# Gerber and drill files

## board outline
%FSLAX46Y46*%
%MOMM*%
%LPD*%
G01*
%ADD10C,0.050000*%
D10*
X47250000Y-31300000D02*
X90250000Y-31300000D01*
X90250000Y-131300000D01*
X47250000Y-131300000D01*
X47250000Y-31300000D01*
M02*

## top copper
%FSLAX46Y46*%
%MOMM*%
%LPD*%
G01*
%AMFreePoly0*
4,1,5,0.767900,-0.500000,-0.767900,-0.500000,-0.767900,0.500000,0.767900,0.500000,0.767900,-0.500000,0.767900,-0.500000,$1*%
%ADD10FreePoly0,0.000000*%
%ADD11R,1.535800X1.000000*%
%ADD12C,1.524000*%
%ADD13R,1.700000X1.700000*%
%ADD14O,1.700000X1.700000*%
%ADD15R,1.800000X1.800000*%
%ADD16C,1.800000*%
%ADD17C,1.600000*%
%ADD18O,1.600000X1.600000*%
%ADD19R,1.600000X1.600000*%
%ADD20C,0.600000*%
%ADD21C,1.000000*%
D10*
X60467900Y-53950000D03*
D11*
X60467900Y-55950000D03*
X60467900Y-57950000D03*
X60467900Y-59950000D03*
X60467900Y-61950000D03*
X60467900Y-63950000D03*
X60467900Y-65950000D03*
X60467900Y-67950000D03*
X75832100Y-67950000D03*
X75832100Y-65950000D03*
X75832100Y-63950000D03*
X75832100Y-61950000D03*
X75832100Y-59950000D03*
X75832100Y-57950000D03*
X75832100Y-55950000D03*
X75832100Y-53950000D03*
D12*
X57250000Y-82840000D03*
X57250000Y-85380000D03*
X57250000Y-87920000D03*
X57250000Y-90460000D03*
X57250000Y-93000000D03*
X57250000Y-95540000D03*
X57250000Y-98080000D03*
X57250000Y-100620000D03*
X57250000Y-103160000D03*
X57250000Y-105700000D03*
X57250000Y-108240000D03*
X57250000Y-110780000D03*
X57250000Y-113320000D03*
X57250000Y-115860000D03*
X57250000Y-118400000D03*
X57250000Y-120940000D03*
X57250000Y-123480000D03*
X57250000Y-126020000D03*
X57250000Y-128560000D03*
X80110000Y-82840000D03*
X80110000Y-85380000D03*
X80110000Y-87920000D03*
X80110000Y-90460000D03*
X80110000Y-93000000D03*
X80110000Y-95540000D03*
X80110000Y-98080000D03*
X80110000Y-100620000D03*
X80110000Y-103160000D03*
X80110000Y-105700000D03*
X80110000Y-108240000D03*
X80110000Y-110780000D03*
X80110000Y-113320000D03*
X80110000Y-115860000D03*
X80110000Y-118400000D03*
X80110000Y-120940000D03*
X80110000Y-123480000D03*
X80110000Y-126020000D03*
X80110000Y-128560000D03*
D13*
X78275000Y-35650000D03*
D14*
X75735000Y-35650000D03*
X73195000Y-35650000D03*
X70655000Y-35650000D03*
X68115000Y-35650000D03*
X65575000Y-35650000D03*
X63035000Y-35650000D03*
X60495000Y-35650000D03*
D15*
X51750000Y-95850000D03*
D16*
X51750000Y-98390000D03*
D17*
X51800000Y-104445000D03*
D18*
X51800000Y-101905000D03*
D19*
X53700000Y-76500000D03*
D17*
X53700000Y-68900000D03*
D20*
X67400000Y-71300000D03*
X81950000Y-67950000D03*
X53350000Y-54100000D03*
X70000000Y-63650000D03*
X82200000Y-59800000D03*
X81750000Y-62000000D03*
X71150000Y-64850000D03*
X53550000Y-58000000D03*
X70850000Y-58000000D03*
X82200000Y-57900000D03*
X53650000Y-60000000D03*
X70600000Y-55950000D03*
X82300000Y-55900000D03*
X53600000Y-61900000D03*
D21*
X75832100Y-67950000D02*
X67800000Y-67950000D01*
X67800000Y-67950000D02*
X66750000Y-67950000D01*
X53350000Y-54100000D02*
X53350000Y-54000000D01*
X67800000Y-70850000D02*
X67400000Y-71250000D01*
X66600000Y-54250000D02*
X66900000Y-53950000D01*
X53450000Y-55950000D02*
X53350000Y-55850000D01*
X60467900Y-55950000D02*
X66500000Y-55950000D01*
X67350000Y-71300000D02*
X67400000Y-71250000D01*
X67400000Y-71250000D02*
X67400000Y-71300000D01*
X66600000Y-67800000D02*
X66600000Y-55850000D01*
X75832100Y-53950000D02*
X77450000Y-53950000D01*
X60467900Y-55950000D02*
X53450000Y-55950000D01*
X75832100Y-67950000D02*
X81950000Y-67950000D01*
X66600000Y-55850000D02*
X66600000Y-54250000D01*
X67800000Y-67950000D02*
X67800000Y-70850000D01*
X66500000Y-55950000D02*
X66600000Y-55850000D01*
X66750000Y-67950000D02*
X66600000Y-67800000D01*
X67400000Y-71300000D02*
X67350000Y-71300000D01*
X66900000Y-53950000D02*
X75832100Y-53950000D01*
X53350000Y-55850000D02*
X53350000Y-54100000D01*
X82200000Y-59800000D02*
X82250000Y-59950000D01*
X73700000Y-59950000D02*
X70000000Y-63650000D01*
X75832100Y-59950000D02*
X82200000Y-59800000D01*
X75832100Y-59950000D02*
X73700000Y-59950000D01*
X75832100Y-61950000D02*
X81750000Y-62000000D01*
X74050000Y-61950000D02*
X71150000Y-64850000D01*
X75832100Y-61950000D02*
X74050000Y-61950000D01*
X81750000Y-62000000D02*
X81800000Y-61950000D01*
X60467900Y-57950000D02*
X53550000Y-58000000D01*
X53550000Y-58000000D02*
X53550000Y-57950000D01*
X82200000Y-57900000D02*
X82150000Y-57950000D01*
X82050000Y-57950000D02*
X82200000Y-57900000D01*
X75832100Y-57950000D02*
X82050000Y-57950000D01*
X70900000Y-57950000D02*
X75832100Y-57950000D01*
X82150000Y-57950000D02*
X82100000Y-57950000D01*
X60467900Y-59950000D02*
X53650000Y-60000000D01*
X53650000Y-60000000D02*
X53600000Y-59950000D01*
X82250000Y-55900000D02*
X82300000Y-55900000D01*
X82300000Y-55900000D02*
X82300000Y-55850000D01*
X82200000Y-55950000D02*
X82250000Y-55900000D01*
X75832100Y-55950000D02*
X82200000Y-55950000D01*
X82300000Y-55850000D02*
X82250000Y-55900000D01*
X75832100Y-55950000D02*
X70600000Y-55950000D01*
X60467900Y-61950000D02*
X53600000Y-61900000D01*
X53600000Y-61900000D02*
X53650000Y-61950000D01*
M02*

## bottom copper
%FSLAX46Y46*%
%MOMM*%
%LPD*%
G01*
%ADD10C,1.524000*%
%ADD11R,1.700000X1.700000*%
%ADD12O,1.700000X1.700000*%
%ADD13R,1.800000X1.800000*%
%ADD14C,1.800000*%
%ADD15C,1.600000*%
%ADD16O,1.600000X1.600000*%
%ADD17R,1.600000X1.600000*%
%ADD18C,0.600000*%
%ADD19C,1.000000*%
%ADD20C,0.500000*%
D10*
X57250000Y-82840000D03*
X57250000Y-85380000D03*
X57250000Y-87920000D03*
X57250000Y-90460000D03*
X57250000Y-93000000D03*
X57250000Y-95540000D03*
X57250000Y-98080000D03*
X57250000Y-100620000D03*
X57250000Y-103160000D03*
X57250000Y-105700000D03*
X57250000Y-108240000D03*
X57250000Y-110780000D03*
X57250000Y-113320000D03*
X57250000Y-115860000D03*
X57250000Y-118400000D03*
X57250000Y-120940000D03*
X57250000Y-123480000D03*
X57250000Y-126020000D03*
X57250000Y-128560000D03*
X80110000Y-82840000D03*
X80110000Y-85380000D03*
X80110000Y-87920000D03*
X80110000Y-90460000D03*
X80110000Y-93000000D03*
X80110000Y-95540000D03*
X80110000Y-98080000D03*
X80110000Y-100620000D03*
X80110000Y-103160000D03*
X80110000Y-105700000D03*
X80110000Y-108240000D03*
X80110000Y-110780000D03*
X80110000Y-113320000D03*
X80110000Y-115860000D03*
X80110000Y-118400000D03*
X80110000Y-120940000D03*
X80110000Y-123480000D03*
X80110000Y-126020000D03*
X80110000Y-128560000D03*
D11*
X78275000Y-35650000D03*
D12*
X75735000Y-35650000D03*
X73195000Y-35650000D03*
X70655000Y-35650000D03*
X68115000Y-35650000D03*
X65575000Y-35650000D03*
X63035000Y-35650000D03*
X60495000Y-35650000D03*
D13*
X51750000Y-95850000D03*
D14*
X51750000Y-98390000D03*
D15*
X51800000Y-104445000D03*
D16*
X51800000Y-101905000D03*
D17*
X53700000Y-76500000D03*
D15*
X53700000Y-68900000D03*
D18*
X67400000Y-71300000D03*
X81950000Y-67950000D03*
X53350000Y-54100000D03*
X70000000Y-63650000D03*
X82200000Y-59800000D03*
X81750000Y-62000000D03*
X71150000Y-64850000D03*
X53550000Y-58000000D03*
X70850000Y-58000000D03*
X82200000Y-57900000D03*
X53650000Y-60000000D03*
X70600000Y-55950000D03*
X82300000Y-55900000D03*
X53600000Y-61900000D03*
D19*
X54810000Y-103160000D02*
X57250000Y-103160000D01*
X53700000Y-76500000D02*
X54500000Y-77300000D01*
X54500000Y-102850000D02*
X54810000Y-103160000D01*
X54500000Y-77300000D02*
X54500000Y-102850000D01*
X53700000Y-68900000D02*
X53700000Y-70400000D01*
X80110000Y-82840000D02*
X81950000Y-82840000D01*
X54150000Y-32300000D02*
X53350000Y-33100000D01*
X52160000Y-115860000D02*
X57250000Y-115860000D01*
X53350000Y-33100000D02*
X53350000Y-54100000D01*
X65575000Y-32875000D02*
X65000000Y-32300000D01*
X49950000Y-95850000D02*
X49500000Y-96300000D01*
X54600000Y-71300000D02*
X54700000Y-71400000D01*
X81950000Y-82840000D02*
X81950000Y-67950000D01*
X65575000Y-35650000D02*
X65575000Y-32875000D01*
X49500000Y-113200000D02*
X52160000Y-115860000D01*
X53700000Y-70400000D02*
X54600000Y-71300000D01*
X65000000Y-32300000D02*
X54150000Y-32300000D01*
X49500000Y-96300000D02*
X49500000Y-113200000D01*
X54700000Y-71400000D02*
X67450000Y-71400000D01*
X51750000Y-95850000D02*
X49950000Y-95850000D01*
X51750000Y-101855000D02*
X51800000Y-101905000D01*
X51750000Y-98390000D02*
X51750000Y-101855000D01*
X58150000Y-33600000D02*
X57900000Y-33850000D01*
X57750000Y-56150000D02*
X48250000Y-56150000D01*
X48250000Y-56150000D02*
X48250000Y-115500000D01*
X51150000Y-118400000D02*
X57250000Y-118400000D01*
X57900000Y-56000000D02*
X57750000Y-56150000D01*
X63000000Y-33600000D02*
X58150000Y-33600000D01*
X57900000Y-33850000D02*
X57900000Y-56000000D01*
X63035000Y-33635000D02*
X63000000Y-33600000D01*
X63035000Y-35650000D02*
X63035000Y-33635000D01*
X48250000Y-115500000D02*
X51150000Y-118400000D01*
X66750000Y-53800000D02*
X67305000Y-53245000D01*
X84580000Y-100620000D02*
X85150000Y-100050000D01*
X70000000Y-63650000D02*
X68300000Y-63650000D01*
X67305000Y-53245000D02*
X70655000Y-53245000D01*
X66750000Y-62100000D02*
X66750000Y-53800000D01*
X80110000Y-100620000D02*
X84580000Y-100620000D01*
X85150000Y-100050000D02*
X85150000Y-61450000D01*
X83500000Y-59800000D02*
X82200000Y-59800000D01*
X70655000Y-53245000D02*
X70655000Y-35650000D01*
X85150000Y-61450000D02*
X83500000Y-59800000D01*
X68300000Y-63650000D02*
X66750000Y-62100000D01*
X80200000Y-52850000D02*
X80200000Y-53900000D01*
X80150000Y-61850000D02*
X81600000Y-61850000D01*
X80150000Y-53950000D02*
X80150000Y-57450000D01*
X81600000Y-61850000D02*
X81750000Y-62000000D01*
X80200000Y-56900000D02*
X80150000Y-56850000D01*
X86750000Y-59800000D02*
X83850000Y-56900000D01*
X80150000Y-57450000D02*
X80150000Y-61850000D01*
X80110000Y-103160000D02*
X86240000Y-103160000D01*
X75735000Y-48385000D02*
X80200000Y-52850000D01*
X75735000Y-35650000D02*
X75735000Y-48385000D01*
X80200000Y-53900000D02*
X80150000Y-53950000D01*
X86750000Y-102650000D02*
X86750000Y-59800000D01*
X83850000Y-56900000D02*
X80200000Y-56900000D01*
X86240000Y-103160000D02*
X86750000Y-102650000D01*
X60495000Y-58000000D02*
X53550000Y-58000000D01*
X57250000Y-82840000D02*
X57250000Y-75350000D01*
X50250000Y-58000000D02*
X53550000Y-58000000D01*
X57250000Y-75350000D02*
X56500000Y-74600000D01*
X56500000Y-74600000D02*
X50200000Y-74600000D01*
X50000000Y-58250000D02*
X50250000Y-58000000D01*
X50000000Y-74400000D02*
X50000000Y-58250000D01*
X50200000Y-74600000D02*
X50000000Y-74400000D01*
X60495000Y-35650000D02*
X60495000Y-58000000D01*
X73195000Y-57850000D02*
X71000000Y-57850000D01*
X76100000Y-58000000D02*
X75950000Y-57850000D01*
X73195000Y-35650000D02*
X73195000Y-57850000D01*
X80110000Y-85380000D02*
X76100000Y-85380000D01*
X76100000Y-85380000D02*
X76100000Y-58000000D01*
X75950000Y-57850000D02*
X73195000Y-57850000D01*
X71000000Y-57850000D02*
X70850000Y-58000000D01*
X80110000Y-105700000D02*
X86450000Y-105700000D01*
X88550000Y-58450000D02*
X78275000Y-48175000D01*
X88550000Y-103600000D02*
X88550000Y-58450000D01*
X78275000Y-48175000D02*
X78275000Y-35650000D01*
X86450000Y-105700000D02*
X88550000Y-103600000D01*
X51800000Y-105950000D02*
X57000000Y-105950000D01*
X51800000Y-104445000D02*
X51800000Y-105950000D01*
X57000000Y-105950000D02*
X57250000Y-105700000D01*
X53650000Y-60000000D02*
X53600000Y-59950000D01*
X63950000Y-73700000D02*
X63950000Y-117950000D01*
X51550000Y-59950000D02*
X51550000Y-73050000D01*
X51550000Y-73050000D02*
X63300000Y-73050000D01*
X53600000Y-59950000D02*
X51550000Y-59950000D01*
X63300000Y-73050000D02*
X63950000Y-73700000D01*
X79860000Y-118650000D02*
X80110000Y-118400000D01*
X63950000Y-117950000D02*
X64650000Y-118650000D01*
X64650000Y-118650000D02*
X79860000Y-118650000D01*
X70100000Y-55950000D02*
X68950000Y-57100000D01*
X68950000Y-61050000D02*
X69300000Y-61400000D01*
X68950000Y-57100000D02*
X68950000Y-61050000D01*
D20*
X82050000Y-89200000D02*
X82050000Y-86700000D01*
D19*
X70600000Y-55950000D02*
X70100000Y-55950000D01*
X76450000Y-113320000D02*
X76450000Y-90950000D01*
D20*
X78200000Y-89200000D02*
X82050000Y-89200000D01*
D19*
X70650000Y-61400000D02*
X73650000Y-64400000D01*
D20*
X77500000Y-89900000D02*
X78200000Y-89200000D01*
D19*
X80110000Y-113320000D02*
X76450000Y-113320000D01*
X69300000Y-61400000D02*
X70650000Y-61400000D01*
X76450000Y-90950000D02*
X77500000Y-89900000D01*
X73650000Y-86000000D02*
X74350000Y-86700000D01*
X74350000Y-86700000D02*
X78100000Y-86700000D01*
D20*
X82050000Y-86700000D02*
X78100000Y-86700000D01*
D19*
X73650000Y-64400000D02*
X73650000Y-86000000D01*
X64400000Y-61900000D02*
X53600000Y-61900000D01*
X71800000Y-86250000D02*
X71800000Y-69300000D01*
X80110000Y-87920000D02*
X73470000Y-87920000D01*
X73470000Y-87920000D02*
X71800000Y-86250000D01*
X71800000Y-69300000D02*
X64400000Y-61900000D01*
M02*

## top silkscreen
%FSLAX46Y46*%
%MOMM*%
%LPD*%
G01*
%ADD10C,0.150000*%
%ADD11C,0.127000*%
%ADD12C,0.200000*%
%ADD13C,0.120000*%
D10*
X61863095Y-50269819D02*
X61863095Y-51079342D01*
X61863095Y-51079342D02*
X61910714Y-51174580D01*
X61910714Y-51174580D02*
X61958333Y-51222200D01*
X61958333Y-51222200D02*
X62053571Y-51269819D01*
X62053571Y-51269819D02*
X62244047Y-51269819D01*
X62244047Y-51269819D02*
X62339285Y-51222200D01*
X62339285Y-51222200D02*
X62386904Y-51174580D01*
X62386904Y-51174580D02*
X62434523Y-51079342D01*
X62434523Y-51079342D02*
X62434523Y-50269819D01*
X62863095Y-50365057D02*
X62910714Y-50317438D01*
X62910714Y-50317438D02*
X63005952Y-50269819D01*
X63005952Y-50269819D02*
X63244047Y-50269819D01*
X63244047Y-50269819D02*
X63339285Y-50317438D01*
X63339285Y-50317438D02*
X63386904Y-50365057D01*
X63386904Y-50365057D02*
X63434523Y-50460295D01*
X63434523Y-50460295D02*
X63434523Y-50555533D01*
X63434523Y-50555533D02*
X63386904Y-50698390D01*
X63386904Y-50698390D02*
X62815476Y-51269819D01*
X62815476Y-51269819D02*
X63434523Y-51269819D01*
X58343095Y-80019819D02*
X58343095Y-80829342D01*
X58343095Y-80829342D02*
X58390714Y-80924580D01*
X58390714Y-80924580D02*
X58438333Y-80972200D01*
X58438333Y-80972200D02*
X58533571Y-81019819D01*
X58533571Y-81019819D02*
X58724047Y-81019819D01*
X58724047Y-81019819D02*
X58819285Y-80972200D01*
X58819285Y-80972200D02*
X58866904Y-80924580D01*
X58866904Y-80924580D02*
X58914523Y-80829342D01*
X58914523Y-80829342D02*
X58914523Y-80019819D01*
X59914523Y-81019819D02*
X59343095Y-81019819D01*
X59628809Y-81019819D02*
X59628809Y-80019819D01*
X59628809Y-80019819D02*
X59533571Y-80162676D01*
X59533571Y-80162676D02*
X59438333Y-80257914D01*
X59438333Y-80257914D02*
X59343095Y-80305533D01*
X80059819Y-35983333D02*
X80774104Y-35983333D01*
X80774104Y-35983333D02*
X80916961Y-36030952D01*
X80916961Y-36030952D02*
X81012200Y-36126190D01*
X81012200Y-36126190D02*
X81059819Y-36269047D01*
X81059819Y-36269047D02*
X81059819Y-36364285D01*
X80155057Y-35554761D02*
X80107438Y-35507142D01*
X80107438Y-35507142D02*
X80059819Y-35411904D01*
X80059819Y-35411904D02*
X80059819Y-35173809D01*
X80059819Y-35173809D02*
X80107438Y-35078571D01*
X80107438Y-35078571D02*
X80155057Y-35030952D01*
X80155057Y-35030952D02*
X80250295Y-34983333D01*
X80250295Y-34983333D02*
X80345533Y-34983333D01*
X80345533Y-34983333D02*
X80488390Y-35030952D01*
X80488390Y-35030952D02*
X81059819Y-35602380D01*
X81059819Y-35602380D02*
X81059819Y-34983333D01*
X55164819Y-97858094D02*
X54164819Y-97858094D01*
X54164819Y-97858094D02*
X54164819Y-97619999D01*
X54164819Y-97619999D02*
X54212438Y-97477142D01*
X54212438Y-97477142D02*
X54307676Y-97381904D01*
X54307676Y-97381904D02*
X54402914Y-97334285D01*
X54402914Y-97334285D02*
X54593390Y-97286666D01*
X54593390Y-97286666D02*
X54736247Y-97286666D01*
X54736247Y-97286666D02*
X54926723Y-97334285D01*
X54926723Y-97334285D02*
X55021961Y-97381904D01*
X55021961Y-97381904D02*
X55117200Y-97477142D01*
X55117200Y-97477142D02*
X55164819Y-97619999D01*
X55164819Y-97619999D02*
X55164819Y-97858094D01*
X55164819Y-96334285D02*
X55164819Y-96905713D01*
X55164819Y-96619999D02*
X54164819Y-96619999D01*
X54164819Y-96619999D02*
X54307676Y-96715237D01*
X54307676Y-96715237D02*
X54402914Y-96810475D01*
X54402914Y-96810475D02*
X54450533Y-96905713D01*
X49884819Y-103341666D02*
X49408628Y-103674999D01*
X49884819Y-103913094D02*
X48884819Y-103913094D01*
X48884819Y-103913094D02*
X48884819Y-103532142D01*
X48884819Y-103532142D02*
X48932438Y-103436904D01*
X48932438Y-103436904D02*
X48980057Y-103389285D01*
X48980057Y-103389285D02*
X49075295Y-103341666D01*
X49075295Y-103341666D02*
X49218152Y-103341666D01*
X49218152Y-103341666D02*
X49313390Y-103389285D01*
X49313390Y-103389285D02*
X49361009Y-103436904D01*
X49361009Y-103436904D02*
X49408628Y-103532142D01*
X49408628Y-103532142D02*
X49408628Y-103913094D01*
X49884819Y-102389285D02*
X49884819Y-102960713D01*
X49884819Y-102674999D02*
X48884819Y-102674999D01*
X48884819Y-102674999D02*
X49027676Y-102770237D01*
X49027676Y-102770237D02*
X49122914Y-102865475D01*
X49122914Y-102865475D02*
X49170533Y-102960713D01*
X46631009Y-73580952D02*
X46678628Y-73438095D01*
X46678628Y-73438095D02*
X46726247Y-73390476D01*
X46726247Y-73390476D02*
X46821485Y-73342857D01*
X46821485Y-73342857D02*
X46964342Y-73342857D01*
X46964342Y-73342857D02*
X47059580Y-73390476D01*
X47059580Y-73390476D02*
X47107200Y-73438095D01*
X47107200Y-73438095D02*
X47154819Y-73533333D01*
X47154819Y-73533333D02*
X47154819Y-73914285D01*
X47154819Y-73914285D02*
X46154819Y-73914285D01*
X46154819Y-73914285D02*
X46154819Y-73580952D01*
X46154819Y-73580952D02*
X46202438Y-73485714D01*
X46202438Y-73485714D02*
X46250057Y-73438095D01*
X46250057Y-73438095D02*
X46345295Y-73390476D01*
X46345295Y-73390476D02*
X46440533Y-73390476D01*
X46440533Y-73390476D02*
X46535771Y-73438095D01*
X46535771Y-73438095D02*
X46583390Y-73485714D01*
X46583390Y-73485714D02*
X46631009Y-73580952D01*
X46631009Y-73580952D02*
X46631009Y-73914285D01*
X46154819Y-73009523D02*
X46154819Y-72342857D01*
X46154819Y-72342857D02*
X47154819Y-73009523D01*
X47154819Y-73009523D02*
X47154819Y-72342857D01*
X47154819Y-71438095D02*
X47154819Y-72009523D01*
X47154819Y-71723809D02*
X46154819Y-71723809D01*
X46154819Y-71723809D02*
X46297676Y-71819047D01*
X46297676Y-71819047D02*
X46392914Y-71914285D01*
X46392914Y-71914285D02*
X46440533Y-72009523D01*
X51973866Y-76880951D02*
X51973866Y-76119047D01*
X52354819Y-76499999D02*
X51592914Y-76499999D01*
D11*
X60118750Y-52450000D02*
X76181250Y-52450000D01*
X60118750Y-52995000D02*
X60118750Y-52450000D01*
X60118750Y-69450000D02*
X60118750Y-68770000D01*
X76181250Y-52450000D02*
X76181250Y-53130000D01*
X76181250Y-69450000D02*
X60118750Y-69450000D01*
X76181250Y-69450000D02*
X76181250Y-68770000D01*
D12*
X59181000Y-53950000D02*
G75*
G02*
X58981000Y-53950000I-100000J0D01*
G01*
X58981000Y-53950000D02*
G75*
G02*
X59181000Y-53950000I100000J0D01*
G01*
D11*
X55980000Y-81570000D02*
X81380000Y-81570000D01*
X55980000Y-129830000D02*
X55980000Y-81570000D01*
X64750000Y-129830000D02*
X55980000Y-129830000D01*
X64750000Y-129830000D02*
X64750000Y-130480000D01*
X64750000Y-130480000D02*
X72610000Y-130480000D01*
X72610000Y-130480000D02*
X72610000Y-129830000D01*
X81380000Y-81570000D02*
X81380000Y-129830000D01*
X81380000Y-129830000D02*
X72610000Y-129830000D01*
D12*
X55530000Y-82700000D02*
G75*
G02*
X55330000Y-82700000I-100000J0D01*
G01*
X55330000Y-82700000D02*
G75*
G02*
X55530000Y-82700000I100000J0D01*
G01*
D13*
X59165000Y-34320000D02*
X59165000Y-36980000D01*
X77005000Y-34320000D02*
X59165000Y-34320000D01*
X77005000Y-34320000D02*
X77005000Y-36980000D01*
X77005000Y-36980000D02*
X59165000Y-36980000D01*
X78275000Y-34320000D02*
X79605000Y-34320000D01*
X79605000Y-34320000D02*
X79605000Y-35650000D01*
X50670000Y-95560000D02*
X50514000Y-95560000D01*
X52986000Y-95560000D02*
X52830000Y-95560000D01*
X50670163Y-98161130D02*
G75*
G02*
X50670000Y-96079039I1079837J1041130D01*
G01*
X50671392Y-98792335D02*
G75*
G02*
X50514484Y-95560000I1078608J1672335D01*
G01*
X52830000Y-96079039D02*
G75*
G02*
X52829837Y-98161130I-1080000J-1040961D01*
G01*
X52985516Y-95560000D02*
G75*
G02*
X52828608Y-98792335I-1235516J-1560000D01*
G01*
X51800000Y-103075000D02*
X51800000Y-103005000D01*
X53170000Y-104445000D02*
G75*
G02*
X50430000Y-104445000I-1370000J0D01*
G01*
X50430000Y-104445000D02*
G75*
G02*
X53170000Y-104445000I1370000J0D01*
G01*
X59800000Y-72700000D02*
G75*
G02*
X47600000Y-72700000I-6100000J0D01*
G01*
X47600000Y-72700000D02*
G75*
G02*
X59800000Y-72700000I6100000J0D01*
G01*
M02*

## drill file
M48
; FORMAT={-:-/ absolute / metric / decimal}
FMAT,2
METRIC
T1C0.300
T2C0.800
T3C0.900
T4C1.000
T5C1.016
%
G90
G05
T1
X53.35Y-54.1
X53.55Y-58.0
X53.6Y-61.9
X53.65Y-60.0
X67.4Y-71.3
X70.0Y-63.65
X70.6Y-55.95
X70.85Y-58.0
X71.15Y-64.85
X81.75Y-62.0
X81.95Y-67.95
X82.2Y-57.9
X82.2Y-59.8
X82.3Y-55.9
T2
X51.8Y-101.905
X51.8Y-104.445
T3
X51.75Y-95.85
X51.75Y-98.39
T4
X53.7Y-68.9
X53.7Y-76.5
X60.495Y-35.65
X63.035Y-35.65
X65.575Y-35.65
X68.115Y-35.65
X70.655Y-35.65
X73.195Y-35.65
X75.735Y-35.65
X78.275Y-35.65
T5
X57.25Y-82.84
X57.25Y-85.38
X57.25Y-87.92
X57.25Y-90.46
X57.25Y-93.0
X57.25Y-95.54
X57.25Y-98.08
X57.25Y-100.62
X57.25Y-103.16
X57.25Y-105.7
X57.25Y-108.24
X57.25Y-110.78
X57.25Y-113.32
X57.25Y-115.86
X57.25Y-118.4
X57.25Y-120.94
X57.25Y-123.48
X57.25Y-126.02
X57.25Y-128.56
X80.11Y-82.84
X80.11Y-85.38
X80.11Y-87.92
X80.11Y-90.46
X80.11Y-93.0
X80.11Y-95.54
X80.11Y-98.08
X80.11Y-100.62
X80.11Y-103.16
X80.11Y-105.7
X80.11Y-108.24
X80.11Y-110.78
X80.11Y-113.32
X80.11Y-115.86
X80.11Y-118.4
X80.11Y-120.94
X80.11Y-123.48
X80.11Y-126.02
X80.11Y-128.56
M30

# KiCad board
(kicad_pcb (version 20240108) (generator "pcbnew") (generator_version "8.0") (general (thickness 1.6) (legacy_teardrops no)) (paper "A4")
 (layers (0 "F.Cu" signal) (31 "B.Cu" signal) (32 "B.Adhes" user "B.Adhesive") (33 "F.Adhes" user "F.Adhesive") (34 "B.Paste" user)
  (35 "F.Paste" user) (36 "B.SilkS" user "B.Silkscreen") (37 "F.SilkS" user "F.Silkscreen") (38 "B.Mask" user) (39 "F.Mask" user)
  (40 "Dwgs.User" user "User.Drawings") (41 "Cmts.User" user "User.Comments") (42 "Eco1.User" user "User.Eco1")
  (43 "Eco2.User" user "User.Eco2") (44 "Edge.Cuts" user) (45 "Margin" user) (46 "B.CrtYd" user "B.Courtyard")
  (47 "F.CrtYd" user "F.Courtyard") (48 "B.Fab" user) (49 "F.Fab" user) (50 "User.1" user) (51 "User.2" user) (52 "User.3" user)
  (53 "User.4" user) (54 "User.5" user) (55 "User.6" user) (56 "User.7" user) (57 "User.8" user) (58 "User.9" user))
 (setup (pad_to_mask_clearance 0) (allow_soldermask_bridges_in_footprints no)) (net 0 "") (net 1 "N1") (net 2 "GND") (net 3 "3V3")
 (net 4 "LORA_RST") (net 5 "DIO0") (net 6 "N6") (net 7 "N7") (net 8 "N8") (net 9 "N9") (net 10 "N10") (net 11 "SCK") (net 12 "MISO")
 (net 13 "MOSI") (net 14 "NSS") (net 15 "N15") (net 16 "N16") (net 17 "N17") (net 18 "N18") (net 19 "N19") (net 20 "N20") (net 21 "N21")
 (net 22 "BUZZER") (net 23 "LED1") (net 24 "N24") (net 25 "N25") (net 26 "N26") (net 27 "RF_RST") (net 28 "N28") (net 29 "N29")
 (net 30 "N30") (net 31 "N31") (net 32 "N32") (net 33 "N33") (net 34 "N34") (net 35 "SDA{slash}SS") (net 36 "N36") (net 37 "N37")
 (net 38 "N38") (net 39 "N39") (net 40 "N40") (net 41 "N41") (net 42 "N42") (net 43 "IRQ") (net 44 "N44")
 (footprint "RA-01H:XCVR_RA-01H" (layer "F.Cu") (at 68.15 60.95)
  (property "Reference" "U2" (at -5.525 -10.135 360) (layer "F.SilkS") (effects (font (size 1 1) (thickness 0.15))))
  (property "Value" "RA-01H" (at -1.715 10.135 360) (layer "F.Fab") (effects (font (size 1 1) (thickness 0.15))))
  (fp_line (start -8.03125 -8.5) (end 8.03125 -8.5) (stroke (width 0.127) (type solid)) (layer "F.SilkS"))
  (fp_line (start -8.03125 -7.955) (end -8.03125 -8.5) (stroke (width 0.127) (type solid)) (layer "F.SilkS"))
  (fp_line (start -8.03125 8.5) (end -8.03125 7.82) (stroke (width 0.127) (type solid)) (layer "F.SilkS"))
  (fp_line (start 8.03125 -8.5) (end 8.03125 -7.82) (stroke (width 0.127) (type solid)) (layer "F.SilkS"))
  (fp_line (start 8.03125 8.5) (end -8.03125 8.5) (stroke (width 0.127) (type solid)) (layer "F.SilkS"))
  (fp_line (start 8.03125 8.5) (end 8.03125 7.82) (stroke (width 0.127) (type solid)) (layer "F.SilkS"))
  (fp_circle (center -9.069 -7) (end -8.969 -7) (stroke (width 0.2) (type solid)) (fill none) (layer "F.SilkS"))
  (pad "1" smd custom (at -7.6821 -7) (size 1.5358 1) (layers "F.Cu") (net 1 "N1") (options (clearance outline) (anchor rect)) (primitives))
  (pad "2" smd rect (at -7.6821 -5) (size 1.5358 1) (layers "F.Cu" "F.Paste" "F.Mask") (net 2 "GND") (solder_mask_margin 0.102))
  (pad "3" smd rect (at -7.6821 -3) (size 1.5358 1) (layers "F.Cu" "F.Paste" "F.Mask") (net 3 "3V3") (solder_mask_margin 0.102))
  (pad "4" smd rect (at -7.6821 -1) (size 1.5358 1) (layers "F.Cu" "F.Paste" "F.Mask") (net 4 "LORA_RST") (solder_mask_margin 0.102))
  (pad "5" smd rect (at -7.6821 1) (size 1.5358 1) (layers "F.Cu" "F.Paste" "F.Mask") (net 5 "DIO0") (solder_mask_margin 0.102))
  (pad "6" smd rect (at -7.6821 3) (size 1.5358 1) (layers "F.Cu" "F.Paste" "F.Mask") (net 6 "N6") (solder_mask_margin 0.102))
  (pad "7" smd rect (at -7.6821 5) (size 1.5358 1) (layers "F.Cu" "F.Paste" "F.Mask") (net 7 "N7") (solder_mask_margin 0.102))
  (pad "8" smd rect (at -7.6821 7) (size 1.5358 1) (layers "F.Cu" "F.Paste" "F.Mask") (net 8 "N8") (solder_mask_margin 0.102))
  (pad "9" smd rect (at 7.6821 7) (size 1.5358 1) (layers "F.Cu" "F.Paste" "F.Mask") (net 2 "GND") (solder_mask_margin 0.102))
  (pad "10" smd rect (at 7.6821 5) (size 1.5358 1) (layers "F.Cu" "F.Paste" "F.Mask") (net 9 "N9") (solder_mask_margin 0.102))
  (pad "11" smd rect (at 7.6821 3) (size 1.5358 1) (layers "F.Cu" "F.Paste" "F.Mask") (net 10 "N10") (solder_mask_margin 0.102))
  (pad "12" smd rect (at 7.6821 1) (size 1.5358 1) (layers "F.Cu" "F.Paste" "F.Mask") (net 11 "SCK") (solder_mask_margin 0.102))
  (pad "13" smd rect (at 7.6821 -1) (size 1.5358 1) (layers "F.Cu" "F.Paste" "F.Mask") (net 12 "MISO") (solder_mask_margin 0.102))
  (pad "14" smd rect (at 7.6821 -3) (size 1.5358 1) (layers "F.Cu" "F.Paste" "F.Mask") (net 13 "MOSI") (solder_mask_margin 0.102))
  (pad "15" smd rect (at 7.6821 -5) (size 1.5358 1) (layers "F.Cu" "F.Paste" "F.Mask") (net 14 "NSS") (solder_mask_margin 0.102))
  (pad "16" smd rect (at 7.6821 -7) (size 1.5358 1) (layers "F.Cu" "F.Paste" "F.Mask") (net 2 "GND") (solder_mask_margin 0.102)))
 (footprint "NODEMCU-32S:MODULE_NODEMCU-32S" (layer "F.Cu") (at 68.68 105.7)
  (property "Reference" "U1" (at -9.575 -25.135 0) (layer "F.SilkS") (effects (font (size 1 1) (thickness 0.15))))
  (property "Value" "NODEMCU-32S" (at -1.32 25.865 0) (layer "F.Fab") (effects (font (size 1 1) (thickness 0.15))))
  (fp_line (start -12.7 -24.13) (end 12.7 -24.13) (stroke (width 0.127) (type solid)) (layer "F.SilkS"))
  (fp_line (start -12.7 24.13) (end -12.7 -24.13) (stroke (width 0.127) (type solid)) (layer "F.SilkS"))
  (fp_line (start -3.93 24.13) (end -12.7 24.13) (stroke (width 0.127) (type solid)) (layer "F.SilkS"))
  (fp_line (start -3.93 24.13) (end -3.93 24.78) (stroke (width 0.127) (type solid)) (layer "F.SilkS"))
  (fp_line (start -3.93 24.78) (end 3.93 24.78) (stroke (width 0.127) (type solid)) (layer "F.SilkS"))
  (fp_line (start 3.93 24.78) (end 3.93 24.13) (stroke (width 0.127) (type solid)) (layer "F.SilkS"))
  (fp_line (start 12.7 -24.13) (end 12.7 24.13) (stroke (width 0.127) (type solid)) (layer "F.SilkS"))
  (fp_line (start 12.7 24.13) (end 3.93 24.13) (stroke (width 0.127) (type solid)) (layer "F.SilkS"))
  (fp_circle (center -13.25 -23) (end -13.15 -23) (stroke (width 0.2) (type solid)) (fill none) (layer "F.SilkS"))
  (pad "J1_1" thru_hole circle (at -11.43 -22.86) (size 1.524 1.524) (drill 1.016) (layers "*.Cu" "*.Mask") (remove_unused_layers no)
   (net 3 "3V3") (solder_mask_margin 0.102))
  (pad "J1_2" thru_hole circle (at -11.43 -20.32) (size 1.524 1.524) (drill 1.016) (layers "*.Cu" "*.Mask") (remove_unused_layers no)
   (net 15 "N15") (solder_mask_margin 0.102))
  (pad "J1_3" thru_hole circle (at -11.43 -17.78) (size 1.524 1.524) (drill 1.016) (layers "*.Cu" "*.Mask") (remove_unused_layers no)
   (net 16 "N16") (solder_mask_margin 0.102))
  (pad "J1_4" thru_hole circle (at -11.43 -15.24) (size 1.524 1.524) (drill 1.016) (layers "*.Cu" "*.Mask") (remove_unused_layers no)
   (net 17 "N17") (solder_mask_margin 0.102))
  (pad "J1_5" thru_hole circle (at -11.43 -12.7) (size 1.524 1.524) (drill 1.016) (layers "*.Cu" "*.Mask") (remove_unused_layers no)
   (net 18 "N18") (solder_mask_margin 0.102))
  (pad "J1_6" thru_hole circle (at -11.43 -10.16) (size 1.524 1.524) (drill 1.016) (layers "*.Cu" "*.Mask") (remove_unused_layers no)
   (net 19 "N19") (solder_mask_margin 0.102))
  (pad "J1_7" thru_hole circle (at -11.43 -7.62) (size 1.524 1.524) (drill 1.016) (layers "*.Cu" "*.Mask") (remove_unused_layers no)
   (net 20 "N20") (solder_mask_margin 0.102))
  (pad "J1_8" thru_hole circle (at -11.43 -5.08) (size 1.524 1.524) (drill 1.016) (layers "*.Cu" "*.Mask") (remove_unused_layers no)
   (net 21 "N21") (solder_mask_margin 0.102))
  (pad "J1_9" thru_hole circle (at -11.43 -2.54) (size 1.524 1.524) (drill 1.016) (layers "*.Cu" "*.Mask") (remove_unused_layers no)
   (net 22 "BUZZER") (solder_mask_margin 0.102))
  (pad "J1_10" thru_hole circle (at -11.43 0) (size 1.524 1.524) (drill 1.016) (layers "*.Cu" "*.Mask") (remove_unused_layers no)
   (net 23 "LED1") (solder_mask_margin 0.102))
  (pad "J1_11" thru_hole circle (at -11.43 2.54) (size 1.524 1.524) (drill 1.016) (layers "*.Cu" "*.Mask") (remove_unused_layers no)
   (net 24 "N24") (solder_mask_margin 0.102))
  (pad "J1_12" thru_hole circle (at -11.43 5.08) (size 1.524 1.524) (drill 1.016) (layers "*.Cu" "*.Mask") (remove_unused_layers no)
   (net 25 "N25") (solder_mask_margin 0.102))
  (pad "J1_13" thru_hole circle (at -11.43 7.62) (size 1.524 1.524) (drill 1.016) (layers "*.Cu" "*.Mask") (remove_unused_layers no)
   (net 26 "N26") (solder_mask_margin 0.102))
  (pad "J1_14" thru_hole circle (at -11.43 10.16) (size 1.524 1.524) (drill 1.016) (layers "*.Cu" "*.Mask") (remove_unused_layers no)
   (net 2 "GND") (solder_mask_margin 0.102))
  (pad "J1_15" thru_hole circle (at -11.43 12.7) (size 1.524 1.524) (drill 1.016) (layers "*.Cu" "*.Mask") (remove_unused_layers no)
   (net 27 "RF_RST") (solder_mask_margin 0.102))
  (pad "J1_16" thru_hole circle (at -11.43 15.24) (size 1.524 1.524) (drill 1.016) (layers "*.Cu" "*.Mask") (remove_unused_layers no)
   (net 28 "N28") (solder_mask_margin 0.102))
  (pad "J1_17" thru_hole circle (at -11.43 17.78) (size 1.524 1.524) (drill 1.016) (layers "*.Cu" "*.Mask") (remove_unused_layers no)
   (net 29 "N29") (solder_mask_margin 0.102))
  (pad "J1_18" thru_hole circle (at -11.43 20.32) (size 1.524 1.524) (drill 1.016) (layers "*.Cu" "*.Mask") (remove_unused_layers no)
   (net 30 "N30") (solder_mask_margin 0.102))
  (pad "J1_19" thru_hole circle (at -11.43 22.86) (size 1.524 1.524) (drill 1.016) (layers "*.Cu" "*.Mask") (remove_unused_layers no)
   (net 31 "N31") (solder_mask_margin 0.102))
  (pad "J2_1" thru_hole circle (at 11.43 -22.86) (size 1.524 1.524) (drill 1.016) (layers "*.Cu" "*.Mask") (remove_unused_layers no)
   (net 2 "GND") (solder_mask_margin 0.102))
  (pad "J2_2" thru_hole circle (at 11.43 -20.32) (size 1.524 1.524) (drill 1.016) (layers "*.Cu" "*.Mask") (remove_unused_layers no)
   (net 13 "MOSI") (solder_mask_margin 0.102))
  (pad "J2_3" thru_hole circle (at 11.43 -17.78) (size 1.524 1.524) (drill 1.016) (layers "*.Cu" "*.Mask") (remove_unused_layers no)
   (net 5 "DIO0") (solder_mask_margin 0.102))
  (pad "J2_4" thru_hole circle (at 11.43 -15.24) (size 1.524 1.524) (drill 1.016) (layers "*.Cu" "*.Mask") (remove_unused_layers no)
   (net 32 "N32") (solder_mask_margin 0.102))
  (pad "J2_5" thru_hole circle (at 11.43 -12.7) (size 1.524 1.524) (drill 1.016) (layers "*.Cu" "*.Mask") (remove_unused_layers no)
   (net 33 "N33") (solder_mask_margin 0.102))
  (pad "J2_6" thru_hole circle (at 11.43 -10.16) (size 1.524 1.524) (drill 1.016) (layers "*.Cu" "*.Mask") (remove_unused_layers no)
   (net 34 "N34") (solder_mask_margin 0.102))
  (pad "J2_7" thru_hole circle (at 11.43 -7.62) (size 1.524 1.524) (drill 1.016) (layers "*.Cu" "*.Mask") (remove_unused_layers no)
   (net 2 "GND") (solder_mask_margin 0.102))
  (pad "J2_8" thru_hole circle (at 11.43 -5.08) (size 1.524 1.524) (drill 1.016) (layers "*.Cu" "*.Mask") (remove_unused_layers no)
   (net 12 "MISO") (solder_mask_margin 0.102))
  (pad "J2_9" thru_hole circle (at 11.43 -2.54) (size 1.524 1.524) (drill 1.016) (layers "*.Cu" "*.Mask") (remove_unused_layers no)
   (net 11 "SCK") (solder_mask_margin 0.102))
  (pad "J2_10" thru_hole circle (at 11.43 0) (size 1.524 1.524) (drill 1.016) (layers "*.Cu" "*.Mask") (remove_unused_layers no)
   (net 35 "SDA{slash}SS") (solder_mask_margin 0.102))
  (pad "J2_11" thru_hole circle (at 11.43 2.54) (size 1.524 1.524) (drill 1.016) (layers "*.Cu" "*.Mask") (remove_unused_layers no)
   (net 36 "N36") (solder_mask_margin 0.102))
  (pad "J2_12" thru_hole circle (at 11.43 5.08) (size 1.524 1.524) (drill 1.016) (layers "*.Cu" "*.Mask") (remove_unused_layers no)
   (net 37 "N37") (solder_mask_margin 0.102))
  (pad "J2_13" thru_hole circle (at 11.43 7.62) (size 1.524 1.524) (drill 1.016) (layers "*.Cu" "*.Mask") (remove_unused_layers no)
   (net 14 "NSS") (solder_mask_margin 0.102))
  (pad "J2_14" thru_hole circle (at 11.43 10.16) (size 1.524 1.524) (drill 1.016) (layers "*.Cu" "*.Mask") (remove_unused_layers no)
   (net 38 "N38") (solder_mask_margin 0.102))
  (pad "J2_15" thru_hole circle (at 11.43 12.7) (size 1.524 1.524) (drill 1.016) (layers "*.Cu" "*.Mask") (remove_unused_layers no)
   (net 4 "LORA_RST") (solder_mask_margin 0.102))
  (pad "J2_16" thru_hole circle (at 11.43 15.24) (size 1.524 1.524) (drill 1.016) (layers "*.Cu" "*.Mask") (remove_unused_layers no)
   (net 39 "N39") (solder_mask_margin 0.102))
  (pad "J2_17" thru_hole circle (at 11.43 17.78) (size 1.524 1.524) (drill 1.016) (layers "*.Cu" "*.Mask") (remove_unused_layers no)
   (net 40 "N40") (solder_mask_margin 0.102))
  (pad "J2_18" thru_hole circle (at 11.43 20.32) (size 1.524 1.524) (drill 1.016) (layers "*.Cu" "*.Mask") (remove_unused_layers no)
   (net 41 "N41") (solder_mask_margin 0.102))
  (pad "J2_19" thru_hole circle (at 11.43 22.86) (size 1.524 1.524) (drill 1.016) (layers "*.Cu" "*.Mask") (remove_unused_layers no)
   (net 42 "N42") (solder_mask_margin 0.102)))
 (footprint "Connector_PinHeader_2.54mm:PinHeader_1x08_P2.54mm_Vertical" (layer "F.Cu") (at 78.275 35.65 -90)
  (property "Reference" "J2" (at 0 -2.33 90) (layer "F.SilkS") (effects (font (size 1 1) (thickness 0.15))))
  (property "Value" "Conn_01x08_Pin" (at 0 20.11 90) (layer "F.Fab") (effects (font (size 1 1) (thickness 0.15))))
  (fp_line (start -1.33 19.11) (end 1.33 19.11) (stroke (width 0.12) (type solid)) (layer "F.SilkS"))
  (fp_line (start -1.33 1.27) (end -1.33 19.11) (stroke (width 0.12) (type solid)) (layer "F.SilkS"))
  (fp_line (start -1.33 1.27) (end 1.33 1.27) (stroke (width 0.12) (type solid)) (layer "F.SilkS"))
  (fp_line (start 1.33 1.27) (end 1.33 19.11) (stroke (width 0.12) (type solid)) (layer "F.SilkS"))
  (fp_line (start -1.33 0) (end -1.33 -1.33) (stroke (width 0.12) (type solid)) (layer "F.SilkS"))
  (fp_line (start -1.33 -1.33) (end 0 -1.33) (stroke (width 0.12) (type solid)) (layer "F.SilkS"))
  (pad "1" thru_hole rect (at 0 0 270) (size 1.7 1.7) (drill 1) (layers "*.Cu" "*.Mask") (remove_unused_layers no) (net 35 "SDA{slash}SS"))
  (pad "2" thru_hole oval (at 0 2.54 270) (size 1.7 1.7) (drill 1) (layers "*.Cu" "*.Mask") (remove_unused_layers no) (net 11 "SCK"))
  (pad "3" thru_hole oval (at 0 5.08 270) (size 1.7 1.7) (drill 1) (layers "*.Cu" "*.Mask") (remove_unused_layers no) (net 13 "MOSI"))
  (pad "4" thru_hole oval (at 0 7.62 270) (size 1.7 1.7) (drill 1) (layers "*.Cu" "*.Mask") (remove_unused_layers no) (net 12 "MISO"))
  (pad "5" thru_hole oval (at 0 10.16 270) (size 1.7 1.7) (drill 1) (layers "*.Cu" "*.Mask") (remove_unused_layers no) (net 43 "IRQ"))
  (pad "6" thru_hole oval (at 0 12.7 270) (size 1.7 1.7) (drill 1) (layers "*.Cu" "*.Mask") (remove_unused_layers no) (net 2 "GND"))
  (pad "7" thru_hole oval (at 0 15.24 270) (size 1.7 1.7) (drill 1) (layers "*.Cu" "*.Mask") (remove_unused_layers no) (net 27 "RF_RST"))
  (pad "8" thru_hole oval (at 0 17.78 270) (size 1.7 1.7) (drill 1) (layers "*.Cu" "*.Mask") (remove_unused_layers no) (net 3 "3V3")))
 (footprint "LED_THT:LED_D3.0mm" (layer "F.Cu") (at 51.75 95.85 -90)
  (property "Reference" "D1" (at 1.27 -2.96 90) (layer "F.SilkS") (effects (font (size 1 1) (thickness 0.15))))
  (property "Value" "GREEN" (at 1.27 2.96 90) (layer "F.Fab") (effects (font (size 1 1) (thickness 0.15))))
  (fp_line (start -0.29 1.08) (end -0.29 1.236) (stroke (width 0.12) (type solid)) (layer "F.SilkS"))
  (fp_line (start -0.29 -1.236) (end -0.29 -1.08) (stroke (width 0.12) (type solid)) (layer "F.SilkS"))
  (fp_arc (start 2.31113 1.079837) (mid 1.270117 1.5) (end 0.229039 1.08) (stroke (width 0.12) (type solid)) (layer "F.SilkS"))
  (fp_arc (start 2.942335 1.078608) (mid 1.366487 1.987659) (end -0.29 1.235516) (stroke (width 0.12) (type solid)) (layer "F.SilkS"))
  (fp_arc (start 0.229039 -1.08) (mid 1.270117 -1.5) (end 2.31113 -1.079837) (stroke (width 0.12) (type solid)) (layer "F.SilkS"))
  (fp_arc (start -0.29 -1.235516) (mid 1.366487 -1.987659) (end 2.942335 -1.078608) (stroke (width 0.12) (type solid)) (layer "F.SilkS"))
  (pad "1" thru_hole rect (at 0 0 270) (size 1.8 1.8) (drill 0.9) (layers "*.Cu" "*.Mask") (remove_unused_layers no) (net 2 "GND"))
  (pad "2" thru_hole circle (at 2.54 0 270) (size 1.8 1.8) (drill 0.9) (layers "*.Cu" "*.Mask") (remove_unused_layers no) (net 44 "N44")))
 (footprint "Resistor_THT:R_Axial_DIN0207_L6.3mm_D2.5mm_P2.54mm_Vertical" (layer "F.Cu") (at 51.8 104.445 90)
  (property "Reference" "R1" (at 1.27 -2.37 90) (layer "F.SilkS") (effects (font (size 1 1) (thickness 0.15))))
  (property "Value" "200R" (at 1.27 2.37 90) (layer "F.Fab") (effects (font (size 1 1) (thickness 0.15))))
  (fp_line (start 1.37 0) (end 1.44 0) (stroke (width 0.12) (type solid)) (layer "F.SilkS"))
  (fp_circle (center 0 0) (end 1.37 0) (stroke (width 0.12) (type solid)) (fill none) (layer "F.SilkS"))
  (pad "1" thru_hole circle (at 0 0 90) (size 1.6 1.6) (drill 0.8) (layers "*.Cu" "*.Mask") (remove_unused_layers no) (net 23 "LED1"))
  (pad "2" thru_hole oval (at 2.54 0 90) (size 1.6 1.6) (drill 0.8) (layers "*.Cu" "*.Mask") (remove_unused_layers no) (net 44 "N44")))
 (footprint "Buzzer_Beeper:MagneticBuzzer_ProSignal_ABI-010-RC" (layer "F.Cu") (at 53.7 76.5 90)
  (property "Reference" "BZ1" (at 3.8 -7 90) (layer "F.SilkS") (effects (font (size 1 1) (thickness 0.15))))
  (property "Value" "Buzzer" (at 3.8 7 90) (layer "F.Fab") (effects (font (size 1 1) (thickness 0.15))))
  (fp_circle (center 3.8 0) (end 9.9 0) (stroke (width 0.12) (type solid)) (fill none) (layer "F.SilkS"))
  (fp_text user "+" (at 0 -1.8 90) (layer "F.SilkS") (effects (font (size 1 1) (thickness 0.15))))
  (pad "1" thru_hole rect (at 0 0 90) (size 1.6 1.6) (drill 1) (layers "*.Cu" "*.Mask") (remove_unused_layers no) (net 22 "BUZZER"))
  (pad "2" thru_hole circle (at 7.6 0 90) (size 1.6 1.6) (drill 1) (layers "*.Cu" "*.Mask") (remove_unused_layers no) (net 2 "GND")))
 (gr_rect (start 47.25 31.3) (end 90.25 131.3) (stroke (width 0.05) (type default)) (fill none) (layer "Edge.Cuts"))
 (segment (start 54.81 103.16) (end 57.25 103.16) (width 1) (layer "B.Cu") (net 22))
 (segment (start 53.7 76.5) (end 54.5 77.3) (width 1) (layer "B.Cu") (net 22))
 (segment (start 54.5 102.85) (end 54.81 103.16) (width 1) (layer "B.Cu") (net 22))
 (segment (start 54.5 77.3) (end 54.5 102.85) (width 1) (layer "B.Cu") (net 22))
 (segment (start 75.8321 67.95) (end 67.8 67.95) (width 1) (layer "F.Cu") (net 2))
 (segment (start 67.8 67.95) (end 66.75 67.95) (width 1) (layer "F.Cu") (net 2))
 (segment (start 53.35 54.1) (end 53.35 54) (width 1) (layer "F.Cu") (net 2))
 (segment (start 67.8 70.85) (end 67.4 71.25) (width 1) (layer "F.Cu") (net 2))
 (segment (start 66.6 54.25) (end 66.9 53.95) (width 1) (layer "F.Cu") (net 2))
 (segment (start 53.45 55.95) (end 53.35 55.85) (width 1) (layer "F.Cu") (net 2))
 (segment (start 60.4679 55.95) (end 66.5 55.95) (width 1) (layer "F.Cu") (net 2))
 (segment (start 67.35 71.3) (end 67.4 71.25) (width 1) (layer "F.Cu") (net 2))
 (segment (start 67.4 71.25) (end 67.4 71.3) (width 1) (layer "F.Cu") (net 2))
 (segment (start 66.6 67.8) (end 66.6 55.85) (width 1) (layer "F.Cu") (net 2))
 (segment (start 75.8321 53.95) (end 77.45 53.95) (width 1) (layer "F.Cu") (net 2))
 (segment (start 60.4679 55.95) (end 53.45 55.95) (width 1) (layer "F.Cu") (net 2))
 (segment (start 75.8321 67.95) (end 81.95 67.95) (width 1) (layer "F.Cu") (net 2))
 (segment (start 66.6 55.85) (end 66.6 54.25) (width 1) (layer "F.Cu") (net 2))
 (segment (start 67.8 67.95) (end 67.8 70.85) (width 1) (layer "F.Cu") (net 2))
 (segment (start 66.5 55.95) (end 66.6 55.85) (width 1) (layer "F.Cu") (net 2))
 (segment (start 66.75 67.95) (end 66.6 67.8) (width 1) (layer "F.Cu") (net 2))
 (segment (start 67.4 71.3) (end 67.35 71.3) (width 1) (layer "F.Cu") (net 2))
 (segment (start 66.9 53.95) (end 75.8321 53.95) (width 1) (layer "F.Cu") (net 2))
 (segment (start 53.35 55.85) (end 53.35 54.1) (width 1) (layer "F.Cu") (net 2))
 (via (at 67.4 71.3) (size 0.6) (drill 0.3) (layers "F.Cu" "B.Cu") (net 2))
 (via (at 81.95 67.95) (size 0.6) (drill 0.3) (layers "F.Cu" "B.Cu") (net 2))
 (via (at 53.35 54.1) (size 0.6) (drill 0.3) (layers "F.Cu" "B.Cu") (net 2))
 (segment (start 53.7 68.9) (end 53.7 70.4) (width 1) (layer "B.Cu") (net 2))
 (segment (start 80.11 82.84) (end 81.95 82.84) (width 1) (layer "B.Cu") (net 2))
 (segment (start 54.15 32.3) (end 53.35 33.1) (width 1) (layer "B.Cu") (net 2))
 (segment (start 52.16 115.86) (end 57.25 115.86) (width 1) (layer "B.Cu") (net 2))
 (segment (start 53.35 33.1) (end 53.35 54.1) (width 1) (layer "B.Cu") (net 2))
 (segment (start 65.575 32.875) (end 65 32.3) (width 1) (layer "B.Cu") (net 2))
 (segment (start 49.95 95.85) (end 49.5 96.3) (width 1) (layer "B.Cu") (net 2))
 (segment (start 54.6 71.3) (end 54.7 71.4) (width 1) (layer "B.Cu") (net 2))
 (segment (start 81.95 82.84) (end 81.95 67.95) (width 1) (layer "B.Cu") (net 2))
 (segment (start 65.575 35.65) (end 65.575 32.875) (width 1) (layer "B.Cu") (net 2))
 (segment (start 49.5 113.2) (end 52.16 115.86) (width 1) (layer "B.Cu") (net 2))
 (segment (start 53.7 70.4) (end 54.6 71.3) (width 1) (layer "B.Cu") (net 2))
 (segment (start 65 32.3) (end 54.15 32.3) (width 1) (layer "B.Cu") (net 2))
 (segment (start 49.5 96.3) (end 49.5 113.2) (width 1) (layer "B.Cu") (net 2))
 (segment (start 54.7 71.4) (end 67.45 71.4) (width 1) (layer "B.Cu") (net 2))
 (segment (start 51.75 95.85) (end 49.95 95.85) (width 1) (layer "B.Cu") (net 2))
 (segment (start 51.75 101.855) (end 51.8 101.905) (width 1) (layer "B.Cu") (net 44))
 (segment (start 51.75 98.39) (end 51.75 101.855) (width 1) (layer "B.Cu") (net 44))
 (segment (start 58.15 33.6) (end 57.9 33.85) (width 1) (layer "B.Cu") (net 27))
 (segment (start 57.75 56.15) (end 48.25 56.15) (width 1) (layer "B.Cu") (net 27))
 (segment (start 48.25 56.15) (end 48.25 115.5) (width 1) (layer "B.Cu") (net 27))
 (segment (start 51.15 118.4) (end 57.25 118.4) (width 1) (layer "B.Cu") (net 27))
 (segment (start 57.9 56) (end 57.75 56.15) (width 1) (layer "B.Cu") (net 27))
 (segment (start 63 33.6) (end 58.15 33.6) (width 1) (layer "B.Cu") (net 27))
 (segment (start 57.9 33.85) (end 57.9 56) (width 1) (layer "B.Cu") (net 27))
 (segment (start 63.035 33.635) (end 63 33.6) (width 1) (layer "B.Cu") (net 27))
 (segment (start 63.035 35.65) (end 63.035 33.635) (width 1) (layer "B.Cu") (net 27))
 (segment (start 48.25 115.5) (end 51.15 118.4) (width 1) (layer "B.Cu") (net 27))
 (segment (start 82.2 59.8) (end 82.25 59.95) (width 1) (layer "F.Cu") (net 12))
 (segment (start 73.7 59.95) (end 70 63.65) (width 1) (layer "F.Cu") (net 12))
 (segment (start 75.8321 59.95) (end 82.2 59.8) (width 1) (layer "F.Cu") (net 12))
 (segment (start 75.8321 59.95) (end 73.7 59.95) (width 1) (layer "F.Cu") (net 12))
 (via (at 70 63.65) (size 0.6) (drill 0.3) (layers "F.Cu" "B.Cu") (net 12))
 (via (at 82.2 59.8) (size 0.6) (drill 0.3) (layers "F.Cu" "B.Cu") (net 12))
 (segment (start 66.75 53.8) (end 67.305 53.245) (width 1) (layer "B.Cu") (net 12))
 (segment (start 84.58 100.62) (end 85.15 100.05) (width 1) (layer "B.Cu") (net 12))
 (segment (start 70 63.65) (end 68.3 63.65) (width 1) (layer "B.Cu") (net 12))
 (segment (start 67.305 53.245) (end 70.655 53.245) (width 1) (layer "B.Cu") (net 12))
 (segment (start 66.75 62.1) (end 66.75 53.8) (width 1) (layer "B.Cu") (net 12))
 (segment (start 80.11 100.62) (end 84.58 100.62) (width 1) (layer "B.Cu") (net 12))
 (segment (start 85.15 100.05) (end 85.15 61.45) (width 1) (layer "B.Cu") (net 12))
 (segment (start 83.5 59.8) (end 82.2 59.8) (width 1) (layer "B.Cu") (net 12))
 (segment (start 70.655 53.245) (end 70.655 35.65) (width 1) (layer "B.Cu") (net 12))
 (segment (start 85.15 61.45) (end 83.5 59.8) (width 1) (layer "B.Cu") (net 12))
 (segment (start 68.3 63.65) (end 66.75 62.1) (width 1) (layer "B.Cu") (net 12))
 (segment (start 75.8321 61.95) (end 81.75 62) (width 1) (layer "F.Cu") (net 11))
 (segment (start 74.05 61.95) (end 71.15 64.85) (width 1) (layer "F.Cu") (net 11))
 (segment (start 75.8321 61.95) (end 74.05 61.95) (width 1) (layer "F.Cu") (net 11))
 (segment (start 81.75 62) (end 81.8 61.95) (width 1) (layer "F.Cu") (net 11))
 (via (at 81.75 62) (size 0.6) (drill 0.3) (layers "F.Cu" "B.Cu") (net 11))
 (via (at 71.15 64.85) (size 0.6) (drill 0.3) (layers "F.Cu" "B.Cu") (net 11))
 (segment (start 80.2 52.85) (end 80.2 53.9) (width 1) (layer "B.Cu") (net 11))
 (segment (start 80.15 61.85) (end 81.6 61.85) (width 1) (layer "B.Cu") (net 11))
 (segment (start 80.15 53.95) (end 80.15 57.45) (width 1) (layer "B.Cu") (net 11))
 (segment (start 81.6 61.85) (end 81.75 62) (width 1) (layer "B.Cu") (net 11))
 (segment (start 80.2 56.9) (end 80.15 56.85) (width 1) (layer "B.Cu") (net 11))
 (segment (start 86.75 59.8) (end 83.85 56.9) (width 1) (layer "B.Cu") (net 11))
 (segment (start 80.15 57.45) (end 80.15 61.85) (width 1) (layer "B.Cu") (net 11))
 (segment (start 80.11 103.16) (end 86.24 103.16) (width 1) (layer "B.Cu") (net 11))
 (segment (start 75.735 48.385) (end 80.2 52.85) (width 1) (layer "B.Cu") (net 11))
 (segment (start 75.735 35.65) (end 75.735 48.385) (width 1) (layer "B.Cu") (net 11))
 (segment (start 80.2 53.9) (end 80.15 53.95) (width 1) (layer "B.Cu") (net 11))
 (segment (start 86.75 102.65) (end 86.75 59.8) (width 1) (layer "B.Cu") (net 11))
 (segment (start 83.85 56.9) (end 80.2 56.9) (width 1) (layer "B.Cu") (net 11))
 (segment (start 86.24 103.16) (end 86.75 102.65) (width 1) (layer "B.Cu") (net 11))
 (segment (start 60.4679 57.95) (end 53.55 58) (width 1) (layer "F.Cu") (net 3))
 (segment (start 53.55 58) (end 53.55 57.95) (width 1) (layer "F.Cu") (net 3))
 (via (at 53.55 58) (size 0.6) (drill 0.3) (layers "F.Cu" "B.Cu") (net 3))
 (segment (start 60.495 58) (end 53.55 58) (width 1) (layer "B.Cu") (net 3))
 (segment (start 57.25 82.84) (end 57.25 75.35) (width 1) (layer "B.Cu") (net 3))
 (segment (start 50.25 58) (end 53.55 58) (width 1) (layer "B.Cu") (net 3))
 (segment (start 57.25 75.35) (end 56.5 74.6) (width 1) (layer "B.Cu") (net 3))
 (segment (start 56.5 74.6) (end 50.2 74.6) (width 1) (layer "B.Cu") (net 3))
 (segment (start 50 58.25) (end 50.25 58) (width 1) (layer "B.Cu") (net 3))
 (segment (start 50 74.4) (end 50 58.25) (width 1) (layer "B.Cu") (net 3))
 (segment (start 50.2 74.6) (end 50 74.4) (width 1) (layer "B.Cu") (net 3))
 (segment (start 60.495 35.65) (end 60.495 58) (width 1) (layer "B.Cu") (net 3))
 (segment (start 82.2 57.9) (end 82.15 57.95) (width 1) (layer "F.Cu") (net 13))
 (segment (start 82.05 57.95) (end 82.2 57.9) (width 1) (layer "F.Cu") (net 13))
 (segment (start 75.8321 57.95) (end 82.05 57.95) (width 1) (layer "F.Cu") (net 13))
 (segment (start 70.9 57.95) (end 75.8321 57.95) (width 1) (layer "F.Cu") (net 13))
 (segment (start 82.15 57.95) (end 82.1 57.95) (width 1) (layer "F.Cu") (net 13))
 (via (at 70.85 58) (size 0.6) (drill 0.3) (layers "F.Cu" "B.Cu") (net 13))
 (via (at 82.2 57.9) (size 0.6) (drill 0.3) (layers "F.Cu" "B.Cu") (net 13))
 (segment (start 73.195 57.85) (end 71 57.85) (width 1) (layer "B.Cu") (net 13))
 (segment (start 76.1 58) (end 75.95 57.85) (width 1) (layer "B.Cu") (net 13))
 (segment (start 73.195 35.65) (end 73.195 57.85) (width 1) (layer "B.Cu") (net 13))
 (segment (start 80.11 85.38) (end 76.1 85.38) (width 1) (layer "B.Cu") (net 13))
 (segment (start 76.1 85.38) (end 76.1 58) (width 1) (layer "B.Cu") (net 13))
 (segment (start 75.95 57.85) (end 73.195 57.85) (width 1) (layer "B.Cu") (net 13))
 (segment (start 71 57.85) (end 70.85 58) (width 1) (layer "B.Cu") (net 13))
 (segment (start 80.11 105.7) (end 86.45 105.7) (width 1) (layer "B.Cu") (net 35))
 (segment (start 88.55 58.45) (end 78.275 48.175) (width 1) (layer "B.Cu") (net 35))
 (segment (start 88.55 103.6) (end 88.55 58.45) (width 1) (layer "B.Cu") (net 35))
 (segment (start 78.275 48.175) (end 78.275 35.65) (width 1) (layer "B.Cu") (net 35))
 (segment (start 86.45 105.7) (end 88.55 103.6) (width 1) (layer "B.Cu") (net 35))
 (segment (start 51.8 105.95) (end 57 105.95) (width 1) (layer "B.Cu") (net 23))
 (segment (start 51.8 104.445) (end 51.8 105.95) (width 1) (layer "B.Cu") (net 23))
 (segment (start 57 105.95) (end 57.25 105.7) (width 1) (layer "B.Cu") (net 23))
 (segment (start 60.4679 59.95) (end 53.65 60) (width 1) (layer "F.Cu") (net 4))
 (segment (start 53.65 60) (end 53.6 59.95) (width 1) (layer "F.Cu") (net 4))
 (via (at 53.65 60) (size 0.6) (drill 0.3) (layers "F.Cu" "B.Cu") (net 4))
 (segment (start 53.65 60) (end 53.6 59.95) (width 1) (layer "B.Cu") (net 4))
 (segment (start 63.95 73.7) (end 63.95 117.95) (width 1) (layer "B.Cu") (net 4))
 (segment (start 51.55 59.95) (end 51.55 73.05) (width 1) (layer "B.Cu") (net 4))
 (segment (start 51.55 73.05) (end 63.3 73.05) (width 1) (layer "B.Cu") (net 4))
 (segment (start 53.6 59.95) (end 51.55 59.95) (width 1) (layer "B.Cu") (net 4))
 (segment (start 63.3 73.05) (end 63.95 73.7) (width 1) (layer "B.Cu") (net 4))
 (segment (start 79.86 118.65) (end 80.11 118.4) (width 1) (layer "B.Cu") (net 4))
 (segment (start 63.95 117.95) (end 64.65 118.65) (width 1) (layer "B.Cu") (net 4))
 (segment (start 64.65 118.65) (end 79.86 118.65) (width 1) (layer "B.Cu") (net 4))
 (segment (start 82.25 55.9) (end 82.3 55.9) (width 1) (layer "F.Cu") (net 14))
 (segment (start 82.3 55.9) (end 82.3 55.85) (width 1) (layer "F.Cu") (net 14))
 (segment (start 82.2 55.95) (end 82.25 55.9) (width 1) (layer "F.Cu") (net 14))
 (segment (start 75.8321 55.95) (end 82.2 55.95) (width 1) (layer "F.Cu") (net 14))
 (segment (start 82.3 55.85) (end 82.25 55.9) (width 1) (layer "F.Cu") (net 14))
 (segment (start 75.8321 55.95) (end 70.6 55.95) (width 1) (layer "F.Cu") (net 14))
 (via (at 70.6 55.95) (size 0.6) (drill 0.3) (layers "F.Cu" "B.Cu") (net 14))
 (via (at 82.3 55.9) (size 0.6) (drill 0.3) (layers "F.Cu" "B.Cu") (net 14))
 (segment (start 70.1 55.95) (end 68.95 57.1) (width 1) (layer "B.Cu") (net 14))
 (segment (start 68.95 61.05) (end 69.3 61.4) (width 1) (layer "B.Cu") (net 14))
 (segment (start 68.95 57.1) (end 68.95 61.05) (width 1) (layer "B.Cu") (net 14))
 (segment (start 82.05 89.2) (end 82.05 86.7) (width 0.5) (layer "B.Cu") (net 14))
 (segment (start 70.6 55.95) (end 70.1 55.95) (width 1) (layer "B.Cu") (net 14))
 (segment (start 76.45 113.32) (end 76.45 90.95) (width 1) (layer "B.Cu") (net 14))
 (segment (start 78.2 89.2) (end 82.05 89.2) (width 0.5) (layer "B.Cu") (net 14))
 (segment (start 70.65 61.4) (end 73.65 64.4) (width 1) (layer "B.Cu") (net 14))
 (segment (start 77.5 89.9) (end 78.2 89.2) (width 0.5) (layer "B.Cu") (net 14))
 (segment (start 80.11 113.32) (end 76.45 113.32) (width 1) (layer "B.Cu") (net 14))
 (segment (start 69.3 61.4) (end 70.65 61.4) (width 1) (layer "B.Cu") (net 14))
 (segment (start 76.45 90.95) (end 77.5 89.9) (width 1) (layer "B.Cu") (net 14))
 (segment (start 73.65 86) (end 74.35 86.7) (width 1) (layer "B.Cu") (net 14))
 (segment (start 74.35 86.7) (end 78.1 86.7) (width 1) (layer "B.Cu") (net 14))
 (segment (start 82.05 86.7) (end 78.1 86.7) (width 0.5) (layer "B.Cu") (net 14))
 (segment (start 73.65 64.4) (end 73.65 86) (width 1) (layer "B.Cu") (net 14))
 (segment (start 60.4679 61.95) (end 53.6 61.9) (width 1) (layer "F.Cu") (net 5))
 (segment (start 53.6 61.9) (end 53.65 61.95) (width 1) (layer "F.Cu") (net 5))
 (via (at 53.6 61.9) (size 0.6) (drill 0.3) (layers "F.Cu" "B.Cu") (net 5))
 (segment (start 64.4 61.9) (end 53.6 61.9) (width 1) (layer "B.Cu") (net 5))
 (segment (start 71.8 86.25) (end 71.8 69.3) (width 1) (layer "B.Cu") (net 5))
 (segment (start 80.11 87.92) (end 73.47 87.92) (width 1) (layer "B.Cu") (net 5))
 (segment (start 73.47 87.92) (end 71.8 86.25) (width 1) (layer "B.Cu") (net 5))
 (segment (start 71.8 69.3) (end 64.4 61.9) (width 1) (layer "B.Cu") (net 5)))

